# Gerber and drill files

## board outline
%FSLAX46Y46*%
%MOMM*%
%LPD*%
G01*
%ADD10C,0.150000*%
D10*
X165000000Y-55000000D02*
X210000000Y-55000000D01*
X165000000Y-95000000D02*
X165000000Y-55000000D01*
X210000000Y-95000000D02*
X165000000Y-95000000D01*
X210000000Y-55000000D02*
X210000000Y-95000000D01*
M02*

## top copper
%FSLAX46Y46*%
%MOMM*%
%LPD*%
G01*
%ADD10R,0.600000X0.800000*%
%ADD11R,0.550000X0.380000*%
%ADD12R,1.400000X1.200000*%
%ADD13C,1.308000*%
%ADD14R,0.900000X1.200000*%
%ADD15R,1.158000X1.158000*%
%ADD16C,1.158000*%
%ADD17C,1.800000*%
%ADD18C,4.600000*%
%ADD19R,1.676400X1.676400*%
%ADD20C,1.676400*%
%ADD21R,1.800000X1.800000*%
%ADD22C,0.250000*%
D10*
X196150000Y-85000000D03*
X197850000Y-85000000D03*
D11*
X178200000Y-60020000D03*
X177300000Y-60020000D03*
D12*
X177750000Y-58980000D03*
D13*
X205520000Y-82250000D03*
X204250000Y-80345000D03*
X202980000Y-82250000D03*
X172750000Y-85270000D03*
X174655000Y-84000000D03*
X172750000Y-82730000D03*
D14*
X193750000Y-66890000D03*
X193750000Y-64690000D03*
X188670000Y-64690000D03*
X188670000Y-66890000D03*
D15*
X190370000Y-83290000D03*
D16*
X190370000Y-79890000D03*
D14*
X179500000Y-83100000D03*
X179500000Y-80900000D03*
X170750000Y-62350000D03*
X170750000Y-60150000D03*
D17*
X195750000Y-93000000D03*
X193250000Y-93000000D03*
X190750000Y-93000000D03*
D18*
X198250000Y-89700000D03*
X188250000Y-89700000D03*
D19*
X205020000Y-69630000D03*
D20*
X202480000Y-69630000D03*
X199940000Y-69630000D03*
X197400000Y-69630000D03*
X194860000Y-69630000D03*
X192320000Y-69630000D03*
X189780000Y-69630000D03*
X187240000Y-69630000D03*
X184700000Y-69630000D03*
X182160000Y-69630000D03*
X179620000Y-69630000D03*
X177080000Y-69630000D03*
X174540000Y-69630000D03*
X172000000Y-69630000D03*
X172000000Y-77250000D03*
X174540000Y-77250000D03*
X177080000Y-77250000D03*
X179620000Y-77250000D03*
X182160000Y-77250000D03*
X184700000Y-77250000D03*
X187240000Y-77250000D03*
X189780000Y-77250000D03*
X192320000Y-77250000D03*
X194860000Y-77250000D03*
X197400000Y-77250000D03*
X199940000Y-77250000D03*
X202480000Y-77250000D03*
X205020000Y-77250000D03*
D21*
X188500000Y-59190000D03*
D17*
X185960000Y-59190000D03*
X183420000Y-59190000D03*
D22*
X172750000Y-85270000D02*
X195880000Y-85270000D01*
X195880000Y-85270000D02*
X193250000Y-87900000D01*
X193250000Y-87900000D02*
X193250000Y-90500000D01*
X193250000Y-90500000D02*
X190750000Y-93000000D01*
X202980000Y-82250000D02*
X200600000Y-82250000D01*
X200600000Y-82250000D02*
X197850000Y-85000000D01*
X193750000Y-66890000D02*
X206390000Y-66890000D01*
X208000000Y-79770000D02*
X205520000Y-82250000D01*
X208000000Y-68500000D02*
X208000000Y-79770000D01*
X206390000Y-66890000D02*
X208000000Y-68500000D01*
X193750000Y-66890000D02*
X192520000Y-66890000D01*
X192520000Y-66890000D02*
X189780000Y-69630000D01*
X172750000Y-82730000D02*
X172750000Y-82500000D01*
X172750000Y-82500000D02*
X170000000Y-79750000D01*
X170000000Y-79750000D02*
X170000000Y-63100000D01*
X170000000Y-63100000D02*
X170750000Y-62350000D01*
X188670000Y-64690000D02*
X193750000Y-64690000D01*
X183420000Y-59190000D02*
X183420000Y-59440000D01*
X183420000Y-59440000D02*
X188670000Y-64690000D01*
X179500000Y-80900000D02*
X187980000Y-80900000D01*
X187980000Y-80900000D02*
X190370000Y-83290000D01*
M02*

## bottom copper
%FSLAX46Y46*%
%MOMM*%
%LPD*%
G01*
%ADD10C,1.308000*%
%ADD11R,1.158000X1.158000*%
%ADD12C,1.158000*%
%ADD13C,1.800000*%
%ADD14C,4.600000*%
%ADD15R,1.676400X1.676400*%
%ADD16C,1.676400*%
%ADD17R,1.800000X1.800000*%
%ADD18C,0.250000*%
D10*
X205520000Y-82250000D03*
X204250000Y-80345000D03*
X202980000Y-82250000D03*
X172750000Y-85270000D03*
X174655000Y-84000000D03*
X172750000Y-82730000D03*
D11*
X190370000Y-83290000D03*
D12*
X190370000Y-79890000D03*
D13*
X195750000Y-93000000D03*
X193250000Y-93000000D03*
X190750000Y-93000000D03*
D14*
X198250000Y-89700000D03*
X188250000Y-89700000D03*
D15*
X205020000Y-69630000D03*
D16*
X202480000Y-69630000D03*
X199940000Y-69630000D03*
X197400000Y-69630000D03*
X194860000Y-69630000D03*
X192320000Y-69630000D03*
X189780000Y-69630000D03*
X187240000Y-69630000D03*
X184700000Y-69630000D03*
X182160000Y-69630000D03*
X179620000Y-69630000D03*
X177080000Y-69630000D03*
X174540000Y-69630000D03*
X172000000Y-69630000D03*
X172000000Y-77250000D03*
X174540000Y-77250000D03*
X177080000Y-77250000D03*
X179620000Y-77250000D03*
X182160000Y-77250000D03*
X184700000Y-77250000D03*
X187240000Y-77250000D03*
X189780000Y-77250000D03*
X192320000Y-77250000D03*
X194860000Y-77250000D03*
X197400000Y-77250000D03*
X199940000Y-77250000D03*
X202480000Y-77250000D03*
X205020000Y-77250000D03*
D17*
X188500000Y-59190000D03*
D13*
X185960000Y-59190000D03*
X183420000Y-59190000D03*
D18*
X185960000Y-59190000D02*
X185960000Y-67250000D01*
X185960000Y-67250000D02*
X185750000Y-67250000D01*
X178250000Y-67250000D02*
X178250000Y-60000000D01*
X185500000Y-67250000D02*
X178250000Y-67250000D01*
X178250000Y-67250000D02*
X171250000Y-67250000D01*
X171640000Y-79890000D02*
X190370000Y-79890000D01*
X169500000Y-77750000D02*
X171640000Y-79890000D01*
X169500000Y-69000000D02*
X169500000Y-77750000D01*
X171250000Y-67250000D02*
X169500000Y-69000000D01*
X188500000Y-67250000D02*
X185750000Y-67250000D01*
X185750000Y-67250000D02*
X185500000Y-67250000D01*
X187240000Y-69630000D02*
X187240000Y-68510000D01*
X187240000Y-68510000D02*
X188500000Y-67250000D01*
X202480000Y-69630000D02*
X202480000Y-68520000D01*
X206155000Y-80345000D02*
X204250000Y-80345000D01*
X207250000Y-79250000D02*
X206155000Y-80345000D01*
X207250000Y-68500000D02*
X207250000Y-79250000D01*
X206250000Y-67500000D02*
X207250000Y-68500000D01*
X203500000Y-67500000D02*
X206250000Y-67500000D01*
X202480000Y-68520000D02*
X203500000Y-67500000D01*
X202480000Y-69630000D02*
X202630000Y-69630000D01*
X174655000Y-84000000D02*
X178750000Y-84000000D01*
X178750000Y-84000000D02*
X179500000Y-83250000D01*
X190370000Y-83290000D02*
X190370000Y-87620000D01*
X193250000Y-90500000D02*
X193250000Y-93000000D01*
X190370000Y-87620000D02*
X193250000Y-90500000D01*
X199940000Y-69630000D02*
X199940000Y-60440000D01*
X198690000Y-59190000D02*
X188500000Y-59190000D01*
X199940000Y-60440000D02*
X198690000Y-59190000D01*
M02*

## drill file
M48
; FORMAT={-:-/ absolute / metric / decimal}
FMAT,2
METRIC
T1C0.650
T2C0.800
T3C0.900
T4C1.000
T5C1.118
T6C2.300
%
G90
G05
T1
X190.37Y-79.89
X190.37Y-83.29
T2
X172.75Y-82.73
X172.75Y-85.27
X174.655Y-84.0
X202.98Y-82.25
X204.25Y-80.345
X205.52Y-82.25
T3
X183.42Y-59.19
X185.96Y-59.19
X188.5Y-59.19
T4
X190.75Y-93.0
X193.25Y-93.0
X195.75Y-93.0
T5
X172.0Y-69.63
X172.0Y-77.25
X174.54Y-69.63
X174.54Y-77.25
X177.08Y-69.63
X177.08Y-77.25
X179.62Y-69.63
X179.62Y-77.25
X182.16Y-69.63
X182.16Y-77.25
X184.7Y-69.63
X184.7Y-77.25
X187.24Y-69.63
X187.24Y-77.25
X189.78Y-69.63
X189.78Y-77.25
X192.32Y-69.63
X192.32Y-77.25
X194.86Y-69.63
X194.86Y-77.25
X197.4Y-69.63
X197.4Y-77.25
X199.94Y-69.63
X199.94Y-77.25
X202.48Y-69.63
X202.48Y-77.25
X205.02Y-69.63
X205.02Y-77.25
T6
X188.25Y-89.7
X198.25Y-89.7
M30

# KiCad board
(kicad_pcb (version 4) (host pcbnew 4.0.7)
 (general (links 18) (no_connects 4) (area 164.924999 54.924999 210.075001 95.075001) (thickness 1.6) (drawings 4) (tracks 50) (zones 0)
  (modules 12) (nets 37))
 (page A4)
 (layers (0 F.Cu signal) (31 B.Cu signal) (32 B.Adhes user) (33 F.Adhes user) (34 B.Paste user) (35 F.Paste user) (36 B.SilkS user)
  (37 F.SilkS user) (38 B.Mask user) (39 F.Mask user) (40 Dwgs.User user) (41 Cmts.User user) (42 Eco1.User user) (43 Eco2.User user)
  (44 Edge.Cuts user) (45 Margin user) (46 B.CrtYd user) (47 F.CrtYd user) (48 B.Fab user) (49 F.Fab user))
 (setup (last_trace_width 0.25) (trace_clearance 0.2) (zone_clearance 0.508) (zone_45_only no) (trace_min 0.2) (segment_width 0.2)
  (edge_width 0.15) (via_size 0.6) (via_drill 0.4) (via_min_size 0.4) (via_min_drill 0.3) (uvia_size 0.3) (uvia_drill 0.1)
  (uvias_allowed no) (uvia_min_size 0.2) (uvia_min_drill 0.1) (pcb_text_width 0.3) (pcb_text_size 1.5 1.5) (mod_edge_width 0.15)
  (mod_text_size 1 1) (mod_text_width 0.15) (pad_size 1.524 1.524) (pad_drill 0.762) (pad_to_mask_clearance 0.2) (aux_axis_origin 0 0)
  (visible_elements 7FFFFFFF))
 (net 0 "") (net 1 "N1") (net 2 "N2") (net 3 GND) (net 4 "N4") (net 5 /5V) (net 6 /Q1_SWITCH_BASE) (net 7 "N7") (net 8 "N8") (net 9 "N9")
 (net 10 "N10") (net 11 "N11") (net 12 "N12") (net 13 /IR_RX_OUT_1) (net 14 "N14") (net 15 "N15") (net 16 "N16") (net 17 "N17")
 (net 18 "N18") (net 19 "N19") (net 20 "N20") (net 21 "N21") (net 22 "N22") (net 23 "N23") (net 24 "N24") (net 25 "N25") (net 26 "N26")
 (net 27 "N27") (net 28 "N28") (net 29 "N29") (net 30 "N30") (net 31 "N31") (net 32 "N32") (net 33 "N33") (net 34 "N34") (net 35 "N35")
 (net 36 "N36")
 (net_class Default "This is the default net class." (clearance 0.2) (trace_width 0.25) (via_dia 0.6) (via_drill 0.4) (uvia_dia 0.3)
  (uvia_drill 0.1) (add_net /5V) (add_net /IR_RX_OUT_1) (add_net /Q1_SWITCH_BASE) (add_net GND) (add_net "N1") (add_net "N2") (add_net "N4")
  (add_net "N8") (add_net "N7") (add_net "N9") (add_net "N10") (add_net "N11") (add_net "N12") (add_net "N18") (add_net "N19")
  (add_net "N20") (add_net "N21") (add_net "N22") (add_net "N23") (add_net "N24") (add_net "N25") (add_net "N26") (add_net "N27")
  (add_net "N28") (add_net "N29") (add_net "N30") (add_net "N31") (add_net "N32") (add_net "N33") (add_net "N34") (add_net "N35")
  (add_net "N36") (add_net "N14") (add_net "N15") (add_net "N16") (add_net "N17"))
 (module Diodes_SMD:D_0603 (layer F.Cu) (at 197 85)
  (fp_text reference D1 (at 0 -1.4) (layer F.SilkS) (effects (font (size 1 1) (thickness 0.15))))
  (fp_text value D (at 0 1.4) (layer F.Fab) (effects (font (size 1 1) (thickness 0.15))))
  (pad 1 smd rect (at -0.85 0) (size 0.6 0.8) (layers F.Cu F.Paste F.Mask) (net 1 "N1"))
  (pad 2 smd rect (at 0.85 0) (size 0.6 0.8) (layers F.Cu F.Paste F.Mask) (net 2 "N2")))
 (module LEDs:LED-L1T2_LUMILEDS (layer F.Cu) (at 177.75 59.5)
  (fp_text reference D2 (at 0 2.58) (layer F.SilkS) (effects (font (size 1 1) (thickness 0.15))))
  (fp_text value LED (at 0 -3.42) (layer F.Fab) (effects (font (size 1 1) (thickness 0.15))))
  (pad 1 smd rect (at 0.45 0.52) (size 0.55 0.38) (layers F.Cu F.Paste F.Mask) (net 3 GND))
  (pad 2 smd rect (at -0.45 0.52) (size 0.55 0.38) (layers F.Cu F.Paste F.Mask) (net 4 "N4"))
  (pad 3 smd rect (at 0 -0.52) (size 1.4 1.2) (layers F.Cu F.Paste F.Mask)))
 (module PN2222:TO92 (layer F.Cu) (at 204.25 82.25)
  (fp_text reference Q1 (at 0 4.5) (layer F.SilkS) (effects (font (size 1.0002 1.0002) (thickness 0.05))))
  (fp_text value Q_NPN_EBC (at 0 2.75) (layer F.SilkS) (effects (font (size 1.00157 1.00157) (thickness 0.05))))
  (pad 3 thru_hole circle (at 1.27 0) (size 1.308 1.308) (drill 0.8) (layers *.Cu *.Mask) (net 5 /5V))
  (pad 2 thru_hole circle (at 0 -1.905) (size 1.308 1.308) (drill 0.8) (layers *.Cu *.Mask) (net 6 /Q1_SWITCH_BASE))
  (pad 1 thru_hole circle (at -1.27 0) (size 1.308 1.308) (drill 0.8) (layers *.Cu *.Mask) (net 2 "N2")))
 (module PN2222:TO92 (layer F.Cu) (at 172.75 84 270)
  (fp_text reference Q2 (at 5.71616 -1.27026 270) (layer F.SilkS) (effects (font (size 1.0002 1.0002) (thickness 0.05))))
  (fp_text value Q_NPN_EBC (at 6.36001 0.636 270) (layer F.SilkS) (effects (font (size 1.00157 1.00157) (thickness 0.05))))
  (pad 3 thru_hole circle (at 1.27 0 270) (size 1.308 1.308) (drill 0.8) (layers *.Cu *.Mask) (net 1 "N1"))
  (pad 2 thru_hole circle (at 0 -1.905 270) (size 1.308 1.308) (drill 0.8) (layers *.Cu *.Mask) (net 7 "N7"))
  (pad 1 thru_hole circle (at -1.27 0 270) (size 1.308 1.308) (drill 0.8) (layers *.Cu *.Mask) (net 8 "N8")))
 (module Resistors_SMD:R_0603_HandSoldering (layer F.Cu) (at 193.75 65.79 90)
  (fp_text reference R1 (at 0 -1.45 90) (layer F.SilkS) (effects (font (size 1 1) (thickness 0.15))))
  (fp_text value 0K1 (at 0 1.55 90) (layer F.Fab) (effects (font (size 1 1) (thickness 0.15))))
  (pad 1 smd rect (at -1.1 0 90) (size 1.2 0.9) (layers F.Cu F.Paste F.Mask) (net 5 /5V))
  (pad 2 smd rect (at 1.1 0 90) (size 1.2 0.9) (layers F.Cu F.Paste F.Mask) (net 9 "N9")))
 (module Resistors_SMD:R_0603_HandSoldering (layer F.Cu) (at 188.67 65.79 270)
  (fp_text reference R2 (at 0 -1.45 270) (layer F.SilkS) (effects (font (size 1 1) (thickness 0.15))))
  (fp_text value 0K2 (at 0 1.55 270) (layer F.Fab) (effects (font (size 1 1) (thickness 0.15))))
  (pad 1 smd rect (at -1.1 0 270) (size 1.2 0.9) (layers F.Cu F.Paste F.Mask) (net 9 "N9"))
  (pad 2 smd rect (at 1.1 0 270) (size 1.2 0.9) (layers F.Cu F.Paste F.Mask) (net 3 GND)))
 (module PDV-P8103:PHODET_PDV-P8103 (layer F.Cu) (at 190.37 81.59 90)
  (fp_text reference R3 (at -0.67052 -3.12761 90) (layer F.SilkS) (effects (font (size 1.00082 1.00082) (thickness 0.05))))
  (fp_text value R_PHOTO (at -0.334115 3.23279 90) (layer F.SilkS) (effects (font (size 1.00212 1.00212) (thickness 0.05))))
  (pad 1 thru_hole rect (at -1.7 0 90) (size 1.158 1.158) (drill 0.65) (layers *.Cu *.Mask) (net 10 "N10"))
  (pad 2 thru_hole circle (at 1.7 0 90) (size 1.158 1.158) (drill 0.65) (layers *.Cu *.Mask) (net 3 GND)))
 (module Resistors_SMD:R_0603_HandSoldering (layer F.Cu) (at 179.5 82 90)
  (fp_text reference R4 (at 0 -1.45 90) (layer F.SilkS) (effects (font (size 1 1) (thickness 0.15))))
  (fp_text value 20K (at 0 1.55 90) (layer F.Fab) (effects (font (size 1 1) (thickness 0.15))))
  (pad 1 smd rect (at -1.1 0 90) (size 1.2 0.9) (layers F.Cu F.Paste F.Mask) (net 7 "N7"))
  (pad 2 smd rect (at 1.1 0 90) (size 1.2 0.9) (layers F.Cu F.Paste F.Mask) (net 10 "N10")))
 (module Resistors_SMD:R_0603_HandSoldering (layer F.Cu) (at 170.75 61.25 90)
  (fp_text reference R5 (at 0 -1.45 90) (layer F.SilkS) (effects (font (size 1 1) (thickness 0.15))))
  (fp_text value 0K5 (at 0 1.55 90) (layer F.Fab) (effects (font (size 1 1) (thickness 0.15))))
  (pad 1 smd rect (at -1.1 0 90) (size 1.2 0.9) (layers F.Cu F.Paste F.Mask) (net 8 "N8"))
  (pad 2 smd rect (at 1.1 0 90) (size 1.2 0.9) (layers F.Cu F.Paste F.Mask) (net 4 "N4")))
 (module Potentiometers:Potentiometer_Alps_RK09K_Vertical (layer F.Cu) (at 190.75 93 270)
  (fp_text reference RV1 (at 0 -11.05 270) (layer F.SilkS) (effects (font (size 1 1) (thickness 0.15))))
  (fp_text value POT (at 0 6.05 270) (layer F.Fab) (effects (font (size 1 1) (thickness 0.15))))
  (pad 3 thru_hole circle (at 0 -5 270) (size 1.8 1.8) (drill 1) (layers *.Cu *.Mask) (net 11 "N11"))
  (pad 2 thru_hole circle (at 0 -2.5 270) (size 1.8 1.8) (drill 1) (layers *.Cu *.Mask) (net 10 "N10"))
  (pad 1 thru_hole circle (at 0 0 270) (size 1.8 1.8) (drill 1) (layers *.Cu *.Mask) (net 1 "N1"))
  (pad 0 thru_hole circle (at -3.3 -7.5 270) (size 4.6 4.6) (drill 2.3) (layers *.Cu *.Mask))
  (pad 0 thru_hole circle (at -3.3 2.5 270) (size 4.6 4.6) (drill 2.3) (layers *.Cu *.Mask)))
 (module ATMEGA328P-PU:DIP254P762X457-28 (layer F.Cu) (at 172 77.25 270)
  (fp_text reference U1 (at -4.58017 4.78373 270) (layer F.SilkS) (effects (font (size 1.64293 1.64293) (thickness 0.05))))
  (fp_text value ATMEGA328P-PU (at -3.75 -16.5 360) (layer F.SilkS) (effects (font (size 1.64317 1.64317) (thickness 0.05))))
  (pad 1 thru_hole rect (at -7.62 -33.02 270) (size 1.6764 1.6764) (drill 1.1176) (layers *.Cu *.Mask) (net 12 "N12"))
  (pad 2 thru_hole circle (at -7.62 -30.48 270) (size 1.6764 1.6764) (drill 1.1176) (layers *.Cu *.Mask) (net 6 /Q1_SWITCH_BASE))
  (pad 3 thru_hole circle (at -7.62 -27.94 270) (size 1.6764 1.6764) (drill 1.1176) (layers *.Cu *.Mask) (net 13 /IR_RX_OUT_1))
  (pad 4 thru_hole circle (at -7.62 -25.4 270) (size 1.6764 1.6764) (drill 1.1176) (layers *.Cu *.Mask) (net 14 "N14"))
  (pad 5 thru_hole circle (at -7.62 -22.86 270) (size 1.6764 1.6764) (drill 1.1176) (layers *.Cu *.Mask) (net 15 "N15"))
  (pad 6 thru_hole circle (at -7.62 -20.32 270) (size 1.6764 1.6764) (drill 1.1176) (layers *.Cu *.Mask) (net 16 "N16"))
  (pad 7 thru_hole circle (at -7.62 -17.78 270) (size 1.6764 1.6764) (drill 1.1176) (layers *.Cu *.Mask) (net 5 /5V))
  (pad 8 thru_hole circle (at -7.62 -15.24 270) (size 1.6764 1.6764) (drill 1.1176) (layers *.Cu *.Mask) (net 3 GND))
  (pad 9 thru_hole circle (at -7.62 -12.7 270) (size 1.6764 1.6764) (drill 1.1176) (layers *.Cu *.Mask) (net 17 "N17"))
  (pad 10 thru_hole circle (at -7.62 -10.16 270) (size 1.6764 1.6764) (drill 1.1176) (layers *.Cu *.Mask) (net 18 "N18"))
  (pad 11 thru_hole circle (at -7.62 -7.62 270) (size 1.6764 1.6764) (drill 1.1176) (layers *.Cu *.Mask) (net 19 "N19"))
  (pad 12 thru_hole circle (at -7.62 -5.08 270) (size 1.6764 1.6764) (drill 1.1176) (layers *.Cu *.Mask) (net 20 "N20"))
  (pad 13 thru_hole circle (at -7.62 -2.54 270) (size 1.6764 1.6764) (drill 1.1176) (layers *.Cu *.Mask) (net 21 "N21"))
  (pad 14 thru_hole circle (at -7.62 0 270) (size 1.6764 1.6764) (drill 1.1176) (layers *.Cu *.Mask) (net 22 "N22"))
  (pad 15 thru_hole circle (at 0 0 270) (size 1.6764 1.6764) (drill 1.1176) (layers *.Cu *.Mask) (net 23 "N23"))
  (pad 16 thru_hole circle (at 0 -2.54 270) (size 1.6764 1.6764) (drill 1.1176) (layers *.Cu *.Mask) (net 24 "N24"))
  (pad 17 thru_hole circle (at 0 -5.08 270) (size 1.6764 1.6764) (drill 1.1176) (layers *.Cu *.Mask) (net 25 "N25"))
  (pad 18 thru_hole circle (at 0 -7.62 270) (size 1.6764 1.6764) (drill 1.1176) (layers *.Cu *.Mask) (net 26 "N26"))
  (pad 19 thru_hole circle (at 0 -10.16 270) (size 1.6764 1.6764) (drill 1.1176) (layers *.Cu *.Mask) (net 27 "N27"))
  (pad 20 thru_hole circle (at 0 -12.7 270) (size 1.6764 1.6764) (drill 1.1176) (layers *.Cu *.Mask) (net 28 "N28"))
  (pad 21 thru_hole circle (at 0 -15.24 270) (size 1.6764 1.6764) (drill 1.1176) (layers *.Cu *.Mask) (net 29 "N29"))
  (pad 22 thru_hole circle (at 0 -17.78 270) (size 1.6764 1.6764) (drill 1.1176) (layers *.Cu *.Mask) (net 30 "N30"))
  (pad 23 thru_hole circle (at 0 -20.32 270) (size 1.6764 1.6764) (drill 1.1176) (layers *.Cu *.Mask) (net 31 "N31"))
  (pad 24 thru_hole circle (at 0 -22.86 270) (size 1.6764 1.6764) (drill 1.1176) (layers *.Cu *.Mask) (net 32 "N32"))
  (pad 25 thru_hole circle (at 0 -25.4 270) (size 1.6764 1.6764) (drill 1.1176) (layers *.Cu *.Mask) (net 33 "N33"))
  (pad 26 thru_hole circle (at 0 -27.94 270) (size 1.6764 1.6764) (drill 1.1176) (layers *.Cu *.Mask) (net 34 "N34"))
  (pad 27 thru_hole circle (at 0 -30.48 270) (size 1.6764 1.6764) (drill 1.1176) (layers *.Cu *.Mask) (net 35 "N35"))
  (pad 28 thru_hole circle (at 0 -33.02 270) (size 1.6764 1.6764) (drill 1.1176) (layers *.Cu *.Mask) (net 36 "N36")))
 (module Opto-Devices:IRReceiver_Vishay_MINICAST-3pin (layer F.Cu) (at 188.5 59.19 180)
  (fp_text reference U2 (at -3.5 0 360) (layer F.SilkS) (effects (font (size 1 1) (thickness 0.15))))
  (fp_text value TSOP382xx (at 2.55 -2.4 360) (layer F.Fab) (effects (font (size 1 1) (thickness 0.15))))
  (pad 1 thru_hole rect (at 0 0 180) (size 1.8 1.8) (drill 0.9) (layers *.Cu *.Mask) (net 13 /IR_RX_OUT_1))
  (pad 2 thru_hole circle (at 2.54 0 180) (size 1.8 1.8) (drill 0.9) (layers *.Cu *.Mask) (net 3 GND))
  (pad 3 thru_hole circle (at 5.08 0 180) (size 1.8 1.8) (drill 0.9) (layers *.Cu *.Mask) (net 9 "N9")))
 (gr_line (start 165 55) (end 210 55) (angle 90) (layer Edge.Cuts) (width 0.15))
 (gr_line (start 165 95) (end 165 55) (angle 90) (layer Edge.Cuts) (width 0.15))
 (gr_line (start 210 95) (end 165 95) (angle 90) (layer Edge.Cuts) (width 0.15))
 (gr_line (start 210 55) (end 210 95) (angle 90) (layer Edge.Cuts) (width 0.15))
 (segment (start 172.75 85.27) (end 195.88 85.27) (width 0.25) (layer F.Cu) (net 1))
 (segment (start 195.88 85.27) (end 193.25 87.9) (width 0.25) (layer F.Cu) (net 1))
 (segment (start 193.25 87.9) (end 193.25 90.5) (width 0.25) (layer F.Cu) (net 1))
 (segment (start 193.25 90.5) (end 190.75 93) (width 0.25) (layer F.Cu) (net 1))
 (segment (start 202.98 82.25) (end 200.6 82.25) (width 0.25) (layer F.Cu) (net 2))
 (segment (start 200.6 82.25) (end 197.85 85) (width 0.25) (layer F.Cu) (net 2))
 (segment (start 185.96 59.19) (end 185.96 67.25) (width 0.25) (layer B.Cu) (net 3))
 (segment (start 185.96 67.25) (end 185.75 67.25) (width 0.25) (layer B.Cu) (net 3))
 (segment (start 178.25 67.25) (end 178.25 60) (width 0.25) (layer B.Cu) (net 3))
 (segment (start 185.5 67.25) (end 178.25 67.25) (width 0.25) (layer B.Cu) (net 3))
 (segment (start 178.25 67.25) (end 171.25 67.25) (width 0.25) (layer B.Cu) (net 3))
 (segment (start 171.64 79.89) (end 190.37 79.89) (width 0.25) (layer B.Cu) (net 3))
 (segment (start 169.5 77.75) (end 171.64 79.89) (width 0.25) (layer B.Cu) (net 3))
 (segment (start 169.5 69) (end 169.5 77.75) (width 0.25) (layer B.Cu) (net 3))
 (segment (start 171.25 67.25) (end 169.5 69) (width 0.25) (layer B.Cu) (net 3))
 (segment (start 188.5 67.25) (end 185.75 67.25) (width 0.25) (layer B.Cu) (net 3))
 (segment (start 185.75 67.25) (end 185.5 67.25) (width 0.25) (layer B.Cu) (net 3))
 (segment (start 187.24 69.63) (end 187.24 68.51) (width 0.25) (layer B.Cu) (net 3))
 (segment (start 187.24 68.51) (end 188.5 67.25) (width 0.25) (layer B.Cu) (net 3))
 (segment (start 193.75 66.89) (end 206.39 66.89) (width 0.25) (layer F.Cu) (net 5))
 (segment (start 208 79.77) (end 205.52 82.25) (width 0.25) (layer F.Cu) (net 5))
 (segment (start 208 68.5) (end 208 79.77) (width 0.25) (layer F.Cu) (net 5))
 (segment (start 206.39 66.89) (end 208 68.5) (width 0.25) (layer F.Cu) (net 5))
 (segment (start 193.75 66.89) (end 192.52 66.89) (width 0.25) (layer F.Cu) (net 5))
 (segment (start 192.52 66.89) (end 189.78 69.63) (width 0.25) (layer F.Cu) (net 5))
 (segment (start 202.48 69.63) (end 202.48 68.52) (width 0.25) (layer B.Cu) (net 6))
 (segment (start 206.155 80.345) (end 204.25 80.345) (width 0.25) (layer B.Cu) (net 6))
 (segment (start 207.25 79.25) (end 206.155 80.345) (width 0.25) (layer B.Cu) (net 6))
 (segment (start 207.25 68.5) (end 207.25 79.25) (width 0.25) (layer B.Cu) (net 6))
 (segment (start 206.25 67.5) (end 207.25 68.5) (width 0.25) (layer B.Cu) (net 6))
 (segment (start 203.5 67.5) (end 206.25 67.5) (width 0.25) (layer B.Cu) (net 6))
 (segment (start 202.48 68.52) (end 203.5 67.5) (width 0.25) (layer B.Cu) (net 6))
 (segment (start 202.48 69.63) (end 202.63 69.63) (width 0.25) (layer B.Cu) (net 6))
 (segment (start 174.655 84) (end 178.75 84) (width 0.25) (layer B.Cu) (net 7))
 (segment (start 178.75 84) (end 179.5 83.25) (width 0.25) (layer B.Cu) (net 7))
 (segment (start 172.75 82.73) (end 172.75 82.5) (width 0.25) (layer F.Cu) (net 8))
 (segment (start 172.75 82.5) (end 170 79.75) (width 0.25) (layer F.Cu) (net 8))
 (segment (start 170 79.75) (end 170 63.1) (width 0.25) (layer F.Cu) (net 8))
 (segment (start 170 63.1) (end 170.75 62.35) (width 0.25) (layer F.Cu) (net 8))
 (segment (start 188.67 64.69) (end 193.75 64.69) (width 0.25) (layer F.Cu) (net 9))
 (segment (start 183.42 59.19) (end 183.42 59.44) (width 0.25) (layer F.Cu) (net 9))
 (segment (start 183.42 59.44) (end 188.67 64.69) (width 0.25) (layer F.Cu) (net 9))
 (segment (start 179.5 80.9) (end 187.98 80.9) (width 0.25) (layer F.Cu) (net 10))
 (segment (start 187.98 80.9) (end 190.37 83.29) (width 0.25) (layer F.Cu) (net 10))
 (segment (start 190.37 83.29) (end 190.37 87.62) (width 0.25) (layer B.Cu) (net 10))
 (segment (start 193.25 90.5) (end 193.25 93) (width 0.25) (layer B.Cu) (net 10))
 (segment (start 190.37 87.62) (end 193.25 90.5) (width 0.25) (layer B.Cu) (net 10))
 (segment (start 199.94 69.63) (end 199.94 60.44) (width 0.25) (layer B.Cu) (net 13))
 (segment (start 198.69 59.19) (end 188.5 59.19) (width 0.25) (layer B.Cu) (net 13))
 (segment (start 199.94 60.44) (end 198.69 59.19) (width 0.25) (layer B.Cu) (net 13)))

